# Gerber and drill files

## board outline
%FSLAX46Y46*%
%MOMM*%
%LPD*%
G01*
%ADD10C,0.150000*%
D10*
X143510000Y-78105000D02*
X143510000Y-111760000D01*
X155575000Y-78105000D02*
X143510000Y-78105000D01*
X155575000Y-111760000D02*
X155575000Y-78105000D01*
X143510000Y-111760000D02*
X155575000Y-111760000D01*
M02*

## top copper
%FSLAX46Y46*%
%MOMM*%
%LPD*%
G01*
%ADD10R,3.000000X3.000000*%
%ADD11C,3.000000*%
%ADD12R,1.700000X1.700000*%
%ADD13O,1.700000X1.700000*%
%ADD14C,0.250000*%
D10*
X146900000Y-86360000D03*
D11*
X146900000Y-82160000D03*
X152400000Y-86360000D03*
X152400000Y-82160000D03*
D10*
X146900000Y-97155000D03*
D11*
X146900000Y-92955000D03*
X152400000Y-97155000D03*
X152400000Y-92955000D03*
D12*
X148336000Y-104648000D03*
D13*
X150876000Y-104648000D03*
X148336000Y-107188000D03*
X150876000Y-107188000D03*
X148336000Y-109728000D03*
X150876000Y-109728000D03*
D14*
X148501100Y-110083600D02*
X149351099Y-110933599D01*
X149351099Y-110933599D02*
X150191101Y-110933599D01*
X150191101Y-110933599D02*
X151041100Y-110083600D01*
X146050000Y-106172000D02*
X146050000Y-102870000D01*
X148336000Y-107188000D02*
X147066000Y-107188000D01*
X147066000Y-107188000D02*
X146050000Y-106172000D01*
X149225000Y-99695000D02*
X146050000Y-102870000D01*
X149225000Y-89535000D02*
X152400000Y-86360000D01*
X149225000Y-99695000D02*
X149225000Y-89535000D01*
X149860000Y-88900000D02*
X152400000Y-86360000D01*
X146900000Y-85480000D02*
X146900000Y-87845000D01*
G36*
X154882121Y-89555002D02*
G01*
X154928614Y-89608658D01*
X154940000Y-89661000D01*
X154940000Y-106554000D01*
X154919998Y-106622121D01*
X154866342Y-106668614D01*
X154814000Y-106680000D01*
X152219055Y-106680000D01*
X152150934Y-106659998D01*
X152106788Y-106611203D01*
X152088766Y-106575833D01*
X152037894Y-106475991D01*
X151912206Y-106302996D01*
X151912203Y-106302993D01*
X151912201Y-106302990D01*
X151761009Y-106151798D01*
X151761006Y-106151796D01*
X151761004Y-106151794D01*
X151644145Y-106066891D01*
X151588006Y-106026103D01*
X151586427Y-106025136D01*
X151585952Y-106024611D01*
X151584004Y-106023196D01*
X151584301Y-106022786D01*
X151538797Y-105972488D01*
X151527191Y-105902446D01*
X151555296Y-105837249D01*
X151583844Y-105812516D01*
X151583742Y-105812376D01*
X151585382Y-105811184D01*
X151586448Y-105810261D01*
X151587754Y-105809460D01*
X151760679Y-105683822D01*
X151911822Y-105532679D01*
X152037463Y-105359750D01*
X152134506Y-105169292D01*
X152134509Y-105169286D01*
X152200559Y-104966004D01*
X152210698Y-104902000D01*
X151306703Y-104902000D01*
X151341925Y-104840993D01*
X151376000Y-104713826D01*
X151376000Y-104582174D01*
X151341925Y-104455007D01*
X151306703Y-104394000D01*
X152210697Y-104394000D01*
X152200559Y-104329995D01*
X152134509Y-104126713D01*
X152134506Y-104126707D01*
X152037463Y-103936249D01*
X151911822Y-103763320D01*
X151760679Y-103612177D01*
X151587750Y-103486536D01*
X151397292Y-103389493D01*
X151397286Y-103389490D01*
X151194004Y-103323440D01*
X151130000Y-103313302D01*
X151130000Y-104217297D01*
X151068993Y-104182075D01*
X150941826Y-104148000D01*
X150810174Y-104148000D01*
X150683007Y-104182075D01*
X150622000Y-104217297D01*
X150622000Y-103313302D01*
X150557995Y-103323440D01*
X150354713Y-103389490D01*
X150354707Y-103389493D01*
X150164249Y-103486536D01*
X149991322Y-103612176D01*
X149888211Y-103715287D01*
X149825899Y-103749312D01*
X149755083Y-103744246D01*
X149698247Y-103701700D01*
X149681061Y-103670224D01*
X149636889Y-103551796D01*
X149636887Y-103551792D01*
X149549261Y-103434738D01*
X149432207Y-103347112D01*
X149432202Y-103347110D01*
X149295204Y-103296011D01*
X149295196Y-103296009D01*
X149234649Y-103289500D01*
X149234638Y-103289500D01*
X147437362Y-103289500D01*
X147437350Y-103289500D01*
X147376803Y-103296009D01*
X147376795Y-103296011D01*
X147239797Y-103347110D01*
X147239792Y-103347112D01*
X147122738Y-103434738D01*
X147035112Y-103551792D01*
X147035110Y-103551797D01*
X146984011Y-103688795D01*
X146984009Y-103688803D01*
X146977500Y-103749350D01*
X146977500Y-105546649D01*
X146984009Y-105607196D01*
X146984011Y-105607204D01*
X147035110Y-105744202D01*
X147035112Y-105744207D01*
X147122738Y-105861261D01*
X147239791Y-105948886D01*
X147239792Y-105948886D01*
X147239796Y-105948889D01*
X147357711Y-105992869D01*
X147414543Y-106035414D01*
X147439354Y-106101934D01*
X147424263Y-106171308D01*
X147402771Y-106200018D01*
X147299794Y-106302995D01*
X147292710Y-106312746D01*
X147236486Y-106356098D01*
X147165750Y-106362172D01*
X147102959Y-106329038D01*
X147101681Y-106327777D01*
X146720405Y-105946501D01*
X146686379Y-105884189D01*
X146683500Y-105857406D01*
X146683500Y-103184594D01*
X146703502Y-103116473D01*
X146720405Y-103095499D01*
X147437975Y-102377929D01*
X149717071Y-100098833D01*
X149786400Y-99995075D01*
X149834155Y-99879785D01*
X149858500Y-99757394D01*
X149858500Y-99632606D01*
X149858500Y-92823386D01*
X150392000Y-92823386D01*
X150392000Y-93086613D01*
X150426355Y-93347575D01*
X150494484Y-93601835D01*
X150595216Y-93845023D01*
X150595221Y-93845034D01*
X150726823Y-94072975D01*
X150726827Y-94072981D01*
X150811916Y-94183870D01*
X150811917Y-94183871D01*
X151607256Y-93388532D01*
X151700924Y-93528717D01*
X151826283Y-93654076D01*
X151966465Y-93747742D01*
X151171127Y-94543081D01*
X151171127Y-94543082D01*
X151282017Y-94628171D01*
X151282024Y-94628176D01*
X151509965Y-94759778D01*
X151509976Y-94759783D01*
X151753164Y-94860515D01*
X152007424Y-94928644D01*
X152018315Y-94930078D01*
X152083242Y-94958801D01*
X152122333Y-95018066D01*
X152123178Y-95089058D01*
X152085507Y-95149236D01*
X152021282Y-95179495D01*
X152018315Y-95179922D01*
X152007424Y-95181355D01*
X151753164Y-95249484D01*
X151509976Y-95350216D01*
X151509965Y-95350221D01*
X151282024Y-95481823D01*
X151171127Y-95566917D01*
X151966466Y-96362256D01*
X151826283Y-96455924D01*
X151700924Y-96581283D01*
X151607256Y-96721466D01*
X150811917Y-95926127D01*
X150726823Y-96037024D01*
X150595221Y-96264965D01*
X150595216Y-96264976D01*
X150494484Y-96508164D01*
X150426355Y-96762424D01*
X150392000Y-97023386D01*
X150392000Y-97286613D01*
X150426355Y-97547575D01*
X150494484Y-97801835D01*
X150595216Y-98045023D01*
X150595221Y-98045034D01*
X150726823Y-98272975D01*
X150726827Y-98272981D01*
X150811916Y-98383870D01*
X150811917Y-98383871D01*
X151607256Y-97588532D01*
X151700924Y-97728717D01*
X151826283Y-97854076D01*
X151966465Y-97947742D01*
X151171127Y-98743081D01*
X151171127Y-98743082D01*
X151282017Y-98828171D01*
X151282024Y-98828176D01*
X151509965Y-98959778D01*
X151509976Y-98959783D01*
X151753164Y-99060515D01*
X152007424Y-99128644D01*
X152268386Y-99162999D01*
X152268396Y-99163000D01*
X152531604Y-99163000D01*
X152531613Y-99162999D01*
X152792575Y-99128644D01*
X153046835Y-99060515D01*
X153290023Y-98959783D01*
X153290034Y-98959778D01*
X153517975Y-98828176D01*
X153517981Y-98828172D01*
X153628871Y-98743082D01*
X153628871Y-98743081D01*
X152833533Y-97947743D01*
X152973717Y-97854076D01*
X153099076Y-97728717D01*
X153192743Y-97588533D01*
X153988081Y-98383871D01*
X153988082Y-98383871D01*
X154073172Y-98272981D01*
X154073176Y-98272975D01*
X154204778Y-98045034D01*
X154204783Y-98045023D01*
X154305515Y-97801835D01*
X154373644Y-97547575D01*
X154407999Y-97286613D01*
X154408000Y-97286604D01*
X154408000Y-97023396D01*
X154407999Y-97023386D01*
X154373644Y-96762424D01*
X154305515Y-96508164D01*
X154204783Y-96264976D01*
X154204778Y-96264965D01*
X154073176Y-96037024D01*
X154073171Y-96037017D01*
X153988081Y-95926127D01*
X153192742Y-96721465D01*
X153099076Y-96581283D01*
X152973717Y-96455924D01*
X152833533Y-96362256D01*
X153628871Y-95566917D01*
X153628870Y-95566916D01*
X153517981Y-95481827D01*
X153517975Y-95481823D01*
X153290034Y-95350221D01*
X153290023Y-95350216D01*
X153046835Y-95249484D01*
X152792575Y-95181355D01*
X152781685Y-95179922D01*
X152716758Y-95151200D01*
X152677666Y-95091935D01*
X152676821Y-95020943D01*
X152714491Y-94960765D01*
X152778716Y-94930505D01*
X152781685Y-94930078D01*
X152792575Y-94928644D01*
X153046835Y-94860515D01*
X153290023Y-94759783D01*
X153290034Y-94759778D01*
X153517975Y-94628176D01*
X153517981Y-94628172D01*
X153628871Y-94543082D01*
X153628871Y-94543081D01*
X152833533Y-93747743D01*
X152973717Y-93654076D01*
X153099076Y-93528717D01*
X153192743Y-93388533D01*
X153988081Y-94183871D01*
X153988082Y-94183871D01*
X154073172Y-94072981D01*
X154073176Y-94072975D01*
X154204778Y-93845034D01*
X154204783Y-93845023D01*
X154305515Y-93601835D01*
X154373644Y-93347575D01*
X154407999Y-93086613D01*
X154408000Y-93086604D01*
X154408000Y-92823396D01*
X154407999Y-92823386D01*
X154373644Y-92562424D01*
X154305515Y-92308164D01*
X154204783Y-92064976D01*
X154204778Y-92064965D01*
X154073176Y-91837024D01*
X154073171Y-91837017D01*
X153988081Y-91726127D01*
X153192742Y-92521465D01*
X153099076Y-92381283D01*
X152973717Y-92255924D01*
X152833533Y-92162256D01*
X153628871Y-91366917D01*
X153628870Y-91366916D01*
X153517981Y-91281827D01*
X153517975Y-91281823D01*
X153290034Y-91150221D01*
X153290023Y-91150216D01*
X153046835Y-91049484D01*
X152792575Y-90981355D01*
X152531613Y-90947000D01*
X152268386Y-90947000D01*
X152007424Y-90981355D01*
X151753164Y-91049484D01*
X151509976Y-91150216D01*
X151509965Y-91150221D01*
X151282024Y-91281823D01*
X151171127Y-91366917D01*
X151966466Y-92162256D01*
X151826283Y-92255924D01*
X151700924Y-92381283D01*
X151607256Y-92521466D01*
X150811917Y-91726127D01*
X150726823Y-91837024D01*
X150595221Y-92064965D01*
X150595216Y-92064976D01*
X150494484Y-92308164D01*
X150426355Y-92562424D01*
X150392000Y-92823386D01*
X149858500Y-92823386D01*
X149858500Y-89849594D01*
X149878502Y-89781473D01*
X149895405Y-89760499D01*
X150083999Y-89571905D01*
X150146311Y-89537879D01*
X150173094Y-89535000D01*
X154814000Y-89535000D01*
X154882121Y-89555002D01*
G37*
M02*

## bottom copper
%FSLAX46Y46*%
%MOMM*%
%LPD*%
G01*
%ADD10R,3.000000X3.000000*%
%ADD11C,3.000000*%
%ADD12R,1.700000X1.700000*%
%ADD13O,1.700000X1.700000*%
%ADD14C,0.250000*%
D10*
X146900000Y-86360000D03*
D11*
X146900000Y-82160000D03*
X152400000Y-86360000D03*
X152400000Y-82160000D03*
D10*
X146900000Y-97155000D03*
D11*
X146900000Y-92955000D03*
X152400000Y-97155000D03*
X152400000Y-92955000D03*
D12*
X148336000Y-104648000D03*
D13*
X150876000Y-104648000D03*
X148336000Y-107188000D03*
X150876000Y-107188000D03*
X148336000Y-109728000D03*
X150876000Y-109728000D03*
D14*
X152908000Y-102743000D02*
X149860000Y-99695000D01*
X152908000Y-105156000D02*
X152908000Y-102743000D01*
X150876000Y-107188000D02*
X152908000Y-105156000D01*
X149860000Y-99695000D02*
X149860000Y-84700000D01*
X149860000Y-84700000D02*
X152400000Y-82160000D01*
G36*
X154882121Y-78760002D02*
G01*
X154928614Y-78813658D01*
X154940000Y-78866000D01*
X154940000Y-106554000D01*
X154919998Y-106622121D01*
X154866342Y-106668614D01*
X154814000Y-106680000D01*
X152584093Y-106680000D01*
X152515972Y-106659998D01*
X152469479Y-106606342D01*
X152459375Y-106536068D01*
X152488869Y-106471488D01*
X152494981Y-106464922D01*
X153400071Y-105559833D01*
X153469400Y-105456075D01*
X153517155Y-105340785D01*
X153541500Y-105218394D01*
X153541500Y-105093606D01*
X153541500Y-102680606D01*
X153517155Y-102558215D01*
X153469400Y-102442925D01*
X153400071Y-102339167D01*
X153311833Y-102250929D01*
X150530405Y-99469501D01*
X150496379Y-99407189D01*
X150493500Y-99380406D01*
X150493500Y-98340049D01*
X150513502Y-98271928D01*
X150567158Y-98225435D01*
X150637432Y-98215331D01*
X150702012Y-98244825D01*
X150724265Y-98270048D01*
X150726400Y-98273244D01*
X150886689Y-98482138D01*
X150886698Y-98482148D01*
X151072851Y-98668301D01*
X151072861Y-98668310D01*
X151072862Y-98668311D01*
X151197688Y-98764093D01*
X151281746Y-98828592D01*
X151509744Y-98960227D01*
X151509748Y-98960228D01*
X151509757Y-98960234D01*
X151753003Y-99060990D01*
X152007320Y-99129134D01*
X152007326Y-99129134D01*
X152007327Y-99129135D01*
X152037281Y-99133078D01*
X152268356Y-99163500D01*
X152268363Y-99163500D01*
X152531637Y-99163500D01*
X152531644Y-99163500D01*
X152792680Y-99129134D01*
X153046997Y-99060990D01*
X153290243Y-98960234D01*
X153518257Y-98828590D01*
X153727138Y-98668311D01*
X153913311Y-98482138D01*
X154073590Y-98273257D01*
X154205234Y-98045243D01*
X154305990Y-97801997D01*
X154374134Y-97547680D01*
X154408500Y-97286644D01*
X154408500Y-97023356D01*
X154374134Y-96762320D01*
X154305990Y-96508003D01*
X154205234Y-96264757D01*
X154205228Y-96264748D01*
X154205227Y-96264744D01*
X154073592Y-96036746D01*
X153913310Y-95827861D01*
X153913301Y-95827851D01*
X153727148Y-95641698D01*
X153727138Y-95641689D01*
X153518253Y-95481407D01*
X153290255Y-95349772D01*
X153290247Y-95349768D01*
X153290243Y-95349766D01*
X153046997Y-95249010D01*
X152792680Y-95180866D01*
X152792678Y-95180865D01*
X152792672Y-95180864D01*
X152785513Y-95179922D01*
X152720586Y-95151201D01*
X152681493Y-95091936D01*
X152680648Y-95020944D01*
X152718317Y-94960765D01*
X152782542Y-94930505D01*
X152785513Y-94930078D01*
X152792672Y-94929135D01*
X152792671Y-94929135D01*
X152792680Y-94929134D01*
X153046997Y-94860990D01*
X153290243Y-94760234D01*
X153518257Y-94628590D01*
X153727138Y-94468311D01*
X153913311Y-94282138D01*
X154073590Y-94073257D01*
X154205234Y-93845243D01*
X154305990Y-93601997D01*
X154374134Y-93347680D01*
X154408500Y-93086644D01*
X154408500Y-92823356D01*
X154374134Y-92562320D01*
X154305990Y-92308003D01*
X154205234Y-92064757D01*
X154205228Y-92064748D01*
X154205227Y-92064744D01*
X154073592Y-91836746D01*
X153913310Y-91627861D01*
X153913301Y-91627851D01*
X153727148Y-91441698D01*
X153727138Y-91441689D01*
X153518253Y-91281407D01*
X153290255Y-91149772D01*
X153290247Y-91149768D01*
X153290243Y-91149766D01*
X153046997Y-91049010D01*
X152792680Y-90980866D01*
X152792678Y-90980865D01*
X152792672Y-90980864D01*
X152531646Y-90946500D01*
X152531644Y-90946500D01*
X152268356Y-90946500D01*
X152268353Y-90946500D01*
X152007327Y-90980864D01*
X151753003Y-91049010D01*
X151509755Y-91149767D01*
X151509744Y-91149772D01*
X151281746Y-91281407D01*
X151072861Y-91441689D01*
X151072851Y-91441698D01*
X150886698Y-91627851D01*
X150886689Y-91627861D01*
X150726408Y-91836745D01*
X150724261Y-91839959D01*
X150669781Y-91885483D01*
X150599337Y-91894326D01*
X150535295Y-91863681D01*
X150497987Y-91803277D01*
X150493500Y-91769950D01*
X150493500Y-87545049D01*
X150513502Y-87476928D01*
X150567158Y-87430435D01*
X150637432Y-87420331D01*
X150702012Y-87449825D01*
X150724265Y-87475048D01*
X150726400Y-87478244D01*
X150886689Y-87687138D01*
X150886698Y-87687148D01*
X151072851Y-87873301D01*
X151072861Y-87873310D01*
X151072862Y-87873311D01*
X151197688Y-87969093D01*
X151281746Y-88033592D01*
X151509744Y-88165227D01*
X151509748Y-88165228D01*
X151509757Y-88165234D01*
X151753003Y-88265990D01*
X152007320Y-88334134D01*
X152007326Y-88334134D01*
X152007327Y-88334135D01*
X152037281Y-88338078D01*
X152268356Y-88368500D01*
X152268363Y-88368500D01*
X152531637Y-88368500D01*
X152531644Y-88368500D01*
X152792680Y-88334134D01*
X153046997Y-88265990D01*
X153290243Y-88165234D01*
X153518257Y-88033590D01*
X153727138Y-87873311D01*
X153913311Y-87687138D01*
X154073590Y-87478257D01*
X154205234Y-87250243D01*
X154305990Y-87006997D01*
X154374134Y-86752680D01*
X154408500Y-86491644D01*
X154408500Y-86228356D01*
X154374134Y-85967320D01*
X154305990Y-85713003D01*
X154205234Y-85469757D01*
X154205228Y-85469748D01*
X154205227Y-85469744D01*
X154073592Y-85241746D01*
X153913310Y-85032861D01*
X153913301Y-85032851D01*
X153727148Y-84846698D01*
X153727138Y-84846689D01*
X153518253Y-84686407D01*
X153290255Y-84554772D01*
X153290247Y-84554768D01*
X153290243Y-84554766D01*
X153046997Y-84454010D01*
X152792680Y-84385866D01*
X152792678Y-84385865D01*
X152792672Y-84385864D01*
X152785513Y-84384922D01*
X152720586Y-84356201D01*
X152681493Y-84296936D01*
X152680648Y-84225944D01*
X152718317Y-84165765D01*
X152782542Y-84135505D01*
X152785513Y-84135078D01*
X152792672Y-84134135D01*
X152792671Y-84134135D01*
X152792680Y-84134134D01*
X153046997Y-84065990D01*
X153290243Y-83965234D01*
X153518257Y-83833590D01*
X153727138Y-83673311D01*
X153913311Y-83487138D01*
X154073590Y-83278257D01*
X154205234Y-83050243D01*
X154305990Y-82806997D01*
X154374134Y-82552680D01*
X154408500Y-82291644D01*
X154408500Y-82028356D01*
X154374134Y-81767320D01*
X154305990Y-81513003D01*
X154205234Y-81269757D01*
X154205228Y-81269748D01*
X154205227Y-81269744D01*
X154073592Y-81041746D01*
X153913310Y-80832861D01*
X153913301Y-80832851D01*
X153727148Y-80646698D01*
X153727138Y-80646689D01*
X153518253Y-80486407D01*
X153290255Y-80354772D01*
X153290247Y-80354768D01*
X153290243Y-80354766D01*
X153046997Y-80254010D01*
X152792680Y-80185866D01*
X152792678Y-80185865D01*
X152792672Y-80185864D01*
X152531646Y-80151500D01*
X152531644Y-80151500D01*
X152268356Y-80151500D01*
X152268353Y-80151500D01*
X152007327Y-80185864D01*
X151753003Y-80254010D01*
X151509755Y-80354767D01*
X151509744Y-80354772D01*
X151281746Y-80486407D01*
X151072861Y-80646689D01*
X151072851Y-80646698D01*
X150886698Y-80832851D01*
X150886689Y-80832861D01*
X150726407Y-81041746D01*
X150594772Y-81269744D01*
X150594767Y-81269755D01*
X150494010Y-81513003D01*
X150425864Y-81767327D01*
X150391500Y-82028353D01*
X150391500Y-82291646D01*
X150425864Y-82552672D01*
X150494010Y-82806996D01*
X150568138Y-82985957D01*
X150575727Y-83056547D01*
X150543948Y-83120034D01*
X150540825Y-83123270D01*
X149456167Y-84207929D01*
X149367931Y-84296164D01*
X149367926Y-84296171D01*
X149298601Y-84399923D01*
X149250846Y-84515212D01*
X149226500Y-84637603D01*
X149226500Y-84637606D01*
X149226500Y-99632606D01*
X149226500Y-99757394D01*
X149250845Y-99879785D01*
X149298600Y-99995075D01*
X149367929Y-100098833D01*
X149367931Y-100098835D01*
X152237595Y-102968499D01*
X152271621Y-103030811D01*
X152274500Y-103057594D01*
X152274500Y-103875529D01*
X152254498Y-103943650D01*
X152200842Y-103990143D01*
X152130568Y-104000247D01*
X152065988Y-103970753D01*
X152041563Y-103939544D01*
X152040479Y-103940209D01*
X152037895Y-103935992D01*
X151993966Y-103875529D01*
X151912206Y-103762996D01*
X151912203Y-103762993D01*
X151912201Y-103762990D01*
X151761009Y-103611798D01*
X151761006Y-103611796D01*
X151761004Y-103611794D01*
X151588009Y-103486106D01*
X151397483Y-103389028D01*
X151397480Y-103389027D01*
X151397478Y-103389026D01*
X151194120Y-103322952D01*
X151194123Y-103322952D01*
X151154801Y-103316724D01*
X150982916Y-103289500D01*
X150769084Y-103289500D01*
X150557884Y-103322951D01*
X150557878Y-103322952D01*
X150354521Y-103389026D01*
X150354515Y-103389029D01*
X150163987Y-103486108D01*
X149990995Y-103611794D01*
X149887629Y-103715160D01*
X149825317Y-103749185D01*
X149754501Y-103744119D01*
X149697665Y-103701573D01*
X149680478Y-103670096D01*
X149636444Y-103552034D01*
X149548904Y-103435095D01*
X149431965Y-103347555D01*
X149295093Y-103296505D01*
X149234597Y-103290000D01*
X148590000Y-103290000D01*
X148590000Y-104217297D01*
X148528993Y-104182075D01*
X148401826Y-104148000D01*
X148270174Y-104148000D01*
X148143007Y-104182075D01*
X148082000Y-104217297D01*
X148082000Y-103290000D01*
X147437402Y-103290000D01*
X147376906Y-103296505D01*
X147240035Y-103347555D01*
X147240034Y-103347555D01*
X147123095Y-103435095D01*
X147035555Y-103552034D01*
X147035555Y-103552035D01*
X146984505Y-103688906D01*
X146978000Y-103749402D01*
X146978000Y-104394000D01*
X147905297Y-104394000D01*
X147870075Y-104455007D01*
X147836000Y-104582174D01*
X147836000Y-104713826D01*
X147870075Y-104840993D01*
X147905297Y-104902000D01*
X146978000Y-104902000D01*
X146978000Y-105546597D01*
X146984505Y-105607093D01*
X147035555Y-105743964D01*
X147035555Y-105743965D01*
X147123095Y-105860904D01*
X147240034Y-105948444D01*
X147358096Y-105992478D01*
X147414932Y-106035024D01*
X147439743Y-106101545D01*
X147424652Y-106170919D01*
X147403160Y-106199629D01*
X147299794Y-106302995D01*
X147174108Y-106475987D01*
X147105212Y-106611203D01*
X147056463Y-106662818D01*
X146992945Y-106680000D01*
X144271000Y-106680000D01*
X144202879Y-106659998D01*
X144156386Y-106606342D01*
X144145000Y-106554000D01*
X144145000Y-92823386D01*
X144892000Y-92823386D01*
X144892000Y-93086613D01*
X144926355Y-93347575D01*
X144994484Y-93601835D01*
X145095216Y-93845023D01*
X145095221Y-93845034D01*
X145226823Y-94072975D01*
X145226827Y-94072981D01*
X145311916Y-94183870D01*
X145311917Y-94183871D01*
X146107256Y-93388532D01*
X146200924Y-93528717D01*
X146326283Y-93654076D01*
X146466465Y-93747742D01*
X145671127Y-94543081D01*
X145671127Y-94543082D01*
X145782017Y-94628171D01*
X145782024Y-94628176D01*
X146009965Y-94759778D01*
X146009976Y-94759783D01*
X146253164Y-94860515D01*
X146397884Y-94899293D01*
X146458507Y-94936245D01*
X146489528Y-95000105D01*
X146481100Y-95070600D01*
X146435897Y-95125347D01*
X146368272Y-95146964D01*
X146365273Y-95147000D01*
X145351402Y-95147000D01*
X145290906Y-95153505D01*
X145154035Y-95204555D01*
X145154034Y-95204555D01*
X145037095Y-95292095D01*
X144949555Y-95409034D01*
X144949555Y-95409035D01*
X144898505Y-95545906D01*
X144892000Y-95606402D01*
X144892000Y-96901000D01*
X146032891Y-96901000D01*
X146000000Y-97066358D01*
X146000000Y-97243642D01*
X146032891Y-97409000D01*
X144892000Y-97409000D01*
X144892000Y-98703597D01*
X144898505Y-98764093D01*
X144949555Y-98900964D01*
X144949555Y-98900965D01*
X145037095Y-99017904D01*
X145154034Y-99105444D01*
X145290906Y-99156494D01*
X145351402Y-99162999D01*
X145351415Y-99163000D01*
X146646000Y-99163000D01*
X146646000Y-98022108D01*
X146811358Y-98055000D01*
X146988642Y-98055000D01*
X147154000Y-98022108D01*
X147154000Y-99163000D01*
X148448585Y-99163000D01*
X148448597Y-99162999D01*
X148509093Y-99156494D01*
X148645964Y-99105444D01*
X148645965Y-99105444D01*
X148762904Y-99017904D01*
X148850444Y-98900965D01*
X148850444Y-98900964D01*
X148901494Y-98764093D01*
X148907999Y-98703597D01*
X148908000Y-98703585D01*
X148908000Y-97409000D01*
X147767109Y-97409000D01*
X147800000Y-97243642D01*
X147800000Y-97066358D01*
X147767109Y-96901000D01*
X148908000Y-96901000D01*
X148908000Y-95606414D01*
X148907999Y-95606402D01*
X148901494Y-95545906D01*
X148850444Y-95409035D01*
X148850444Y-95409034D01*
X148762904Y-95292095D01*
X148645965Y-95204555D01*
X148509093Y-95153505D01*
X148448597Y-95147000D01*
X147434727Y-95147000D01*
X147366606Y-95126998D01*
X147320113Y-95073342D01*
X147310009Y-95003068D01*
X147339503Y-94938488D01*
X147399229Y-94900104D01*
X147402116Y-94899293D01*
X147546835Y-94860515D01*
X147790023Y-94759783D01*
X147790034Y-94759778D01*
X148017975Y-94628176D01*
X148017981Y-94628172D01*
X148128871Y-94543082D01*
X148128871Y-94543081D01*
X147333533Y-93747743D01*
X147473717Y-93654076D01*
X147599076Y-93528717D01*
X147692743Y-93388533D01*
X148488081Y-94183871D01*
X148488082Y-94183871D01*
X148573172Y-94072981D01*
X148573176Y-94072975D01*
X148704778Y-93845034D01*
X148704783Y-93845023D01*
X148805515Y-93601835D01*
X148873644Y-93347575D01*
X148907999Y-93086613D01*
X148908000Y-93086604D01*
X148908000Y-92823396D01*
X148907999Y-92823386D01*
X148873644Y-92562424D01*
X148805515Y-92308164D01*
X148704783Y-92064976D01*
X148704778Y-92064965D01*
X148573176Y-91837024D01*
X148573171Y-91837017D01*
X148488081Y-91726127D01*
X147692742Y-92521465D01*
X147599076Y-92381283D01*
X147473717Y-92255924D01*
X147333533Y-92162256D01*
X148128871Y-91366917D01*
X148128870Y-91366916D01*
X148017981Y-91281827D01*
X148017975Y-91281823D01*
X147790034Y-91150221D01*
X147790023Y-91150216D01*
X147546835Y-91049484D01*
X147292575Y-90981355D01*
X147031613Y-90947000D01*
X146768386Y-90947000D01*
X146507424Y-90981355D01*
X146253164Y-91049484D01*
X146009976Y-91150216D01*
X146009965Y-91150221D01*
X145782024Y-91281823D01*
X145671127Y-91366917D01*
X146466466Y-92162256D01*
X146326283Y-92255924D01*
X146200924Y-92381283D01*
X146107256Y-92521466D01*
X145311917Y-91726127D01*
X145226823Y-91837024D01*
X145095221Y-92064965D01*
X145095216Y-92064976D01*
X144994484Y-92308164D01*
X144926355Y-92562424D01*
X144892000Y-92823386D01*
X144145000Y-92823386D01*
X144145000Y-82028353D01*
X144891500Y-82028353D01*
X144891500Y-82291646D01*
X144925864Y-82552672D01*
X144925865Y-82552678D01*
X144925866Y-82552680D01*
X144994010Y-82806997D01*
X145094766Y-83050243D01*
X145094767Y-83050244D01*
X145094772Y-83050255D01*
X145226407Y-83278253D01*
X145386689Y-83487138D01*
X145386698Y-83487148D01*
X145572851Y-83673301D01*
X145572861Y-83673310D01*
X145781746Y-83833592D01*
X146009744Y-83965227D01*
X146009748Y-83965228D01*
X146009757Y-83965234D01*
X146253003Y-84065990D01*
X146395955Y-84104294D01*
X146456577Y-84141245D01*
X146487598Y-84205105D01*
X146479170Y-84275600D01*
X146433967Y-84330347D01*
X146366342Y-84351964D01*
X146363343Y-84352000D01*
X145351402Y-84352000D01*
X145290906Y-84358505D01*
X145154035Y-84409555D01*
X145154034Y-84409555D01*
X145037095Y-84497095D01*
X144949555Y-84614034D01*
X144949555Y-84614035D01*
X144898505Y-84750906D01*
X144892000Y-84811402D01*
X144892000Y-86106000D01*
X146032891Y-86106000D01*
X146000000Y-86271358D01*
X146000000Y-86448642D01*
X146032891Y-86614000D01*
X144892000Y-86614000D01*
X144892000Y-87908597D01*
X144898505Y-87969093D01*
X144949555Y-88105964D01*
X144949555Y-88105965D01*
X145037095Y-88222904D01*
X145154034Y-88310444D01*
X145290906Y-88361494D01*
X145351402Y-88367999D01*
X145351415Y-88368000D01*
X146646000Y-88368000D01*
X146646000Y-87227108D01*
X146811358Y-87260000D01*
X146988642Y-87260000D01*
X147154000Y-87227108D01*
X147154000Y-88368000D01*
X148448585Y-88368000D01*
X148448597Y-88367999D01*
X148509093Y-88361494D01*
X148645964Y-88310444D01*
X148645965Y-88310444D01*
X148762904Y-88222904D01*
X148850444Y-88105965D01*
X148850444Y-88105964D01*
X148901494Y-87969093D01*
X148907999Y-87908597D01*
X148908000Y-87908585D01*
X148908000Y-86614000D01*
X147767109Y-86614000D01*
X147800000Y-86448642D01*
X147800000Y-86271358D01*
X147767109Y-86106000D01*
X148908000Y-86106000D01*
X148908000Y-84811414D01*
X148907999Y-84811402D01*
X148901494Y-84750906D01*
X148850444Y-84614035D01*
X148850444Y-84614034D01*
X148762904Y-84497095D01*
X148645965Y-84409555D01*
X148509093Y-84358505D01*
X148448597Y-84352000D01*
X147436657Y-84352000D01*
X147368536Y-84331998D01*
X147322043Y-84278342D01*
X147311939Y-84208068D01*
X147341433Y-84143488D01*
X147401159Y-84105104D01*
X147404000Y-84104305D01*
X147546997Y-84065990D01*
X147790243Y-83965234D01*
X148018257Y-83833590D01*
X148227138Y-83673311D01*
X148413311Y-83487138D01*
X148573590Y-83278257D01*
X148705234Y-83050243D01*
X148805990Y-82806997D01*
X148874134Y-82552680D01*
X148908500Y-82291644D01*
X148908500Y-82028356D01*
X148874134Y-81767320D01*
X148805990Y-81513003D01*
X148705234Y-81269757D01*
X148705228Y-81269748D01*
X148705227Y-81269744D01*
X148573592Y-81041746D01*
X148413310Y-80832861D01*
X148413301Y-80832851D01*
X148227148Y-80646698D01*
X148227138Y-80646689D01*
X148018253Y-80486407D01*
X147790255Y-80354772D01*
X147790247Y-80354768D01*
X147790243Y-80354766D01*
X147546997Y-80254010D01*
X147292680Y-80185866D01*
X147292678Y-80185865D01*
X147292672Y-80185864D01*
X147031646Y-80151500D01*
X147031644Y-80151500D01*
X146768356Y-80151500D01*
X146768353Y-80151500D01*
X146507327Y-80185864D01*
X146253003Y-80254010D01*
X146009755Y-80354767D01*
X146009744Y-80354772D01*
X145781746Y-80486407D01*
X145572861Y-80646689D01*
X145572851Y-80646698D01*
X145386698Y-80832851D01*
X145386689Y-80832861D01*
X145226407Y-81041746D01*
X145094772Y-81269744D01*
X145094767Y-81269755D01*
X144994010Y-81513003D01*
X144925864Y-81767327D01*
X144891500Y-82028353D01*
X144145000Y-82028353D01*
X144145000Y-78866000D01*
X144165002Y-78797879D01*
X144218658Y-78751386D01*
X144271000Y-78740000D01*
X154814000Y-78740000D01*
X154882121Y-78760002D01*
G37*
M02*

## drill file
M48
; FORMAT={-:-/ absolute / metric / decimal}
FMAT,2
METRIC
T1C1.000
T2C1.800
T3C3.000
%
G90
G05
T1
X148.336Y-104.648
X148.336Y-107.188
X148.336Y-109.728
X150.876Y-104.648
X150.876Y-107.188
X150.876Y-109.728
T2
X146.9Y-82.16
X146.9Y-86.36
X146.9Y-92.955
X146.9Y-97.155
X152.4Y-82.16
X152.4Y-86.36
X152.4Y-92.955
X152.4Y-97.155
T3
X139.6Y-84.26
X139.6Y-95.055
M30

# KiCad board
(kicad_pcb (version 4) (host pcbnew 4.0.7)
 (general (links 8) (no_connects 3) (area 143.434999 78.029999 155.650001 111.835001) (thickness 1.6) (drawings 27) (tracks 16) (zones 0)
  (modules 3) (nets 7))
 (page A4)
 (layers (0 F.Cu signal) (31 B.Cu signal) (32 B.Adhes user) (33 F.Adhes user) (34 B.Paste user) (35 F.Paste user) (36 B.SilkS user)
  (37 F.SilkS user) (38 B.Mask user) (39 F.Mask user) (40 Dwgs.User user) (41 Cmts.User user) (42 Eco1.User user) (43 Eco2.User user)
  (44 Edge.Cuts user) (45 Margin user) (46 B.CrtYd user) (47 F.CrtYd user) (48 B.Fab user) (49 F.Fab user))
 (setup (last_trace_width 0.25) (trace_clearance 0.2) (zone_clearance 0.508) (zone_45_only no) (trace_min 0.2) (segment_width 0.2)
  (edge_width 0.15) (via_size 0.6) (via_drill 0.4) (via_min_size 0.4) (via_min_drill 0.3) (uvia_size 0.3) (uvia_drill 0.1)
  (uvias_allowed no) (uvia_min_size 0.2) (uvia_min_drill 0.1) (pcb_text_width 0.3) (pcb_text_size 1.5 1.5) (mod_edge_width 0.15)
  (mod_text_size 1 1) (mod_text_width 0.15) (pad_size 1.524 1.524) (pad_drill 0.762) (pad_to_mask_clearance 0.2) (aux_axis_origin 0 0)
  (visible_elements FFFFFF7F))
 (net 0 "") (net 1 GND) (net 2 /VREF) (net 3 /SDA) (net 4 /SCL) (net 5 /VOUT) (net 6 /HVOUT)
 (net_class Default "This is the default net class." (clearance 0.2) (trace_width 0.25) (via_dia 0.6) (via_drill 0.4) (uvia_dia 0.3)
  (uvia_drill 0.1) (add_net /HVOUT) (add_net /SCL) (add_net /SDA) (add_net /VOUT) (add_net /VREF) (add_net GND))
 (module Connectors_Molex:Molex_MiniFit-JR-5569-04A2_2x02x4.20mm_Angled (layer F.Cu) (at 146.9 86.36 90)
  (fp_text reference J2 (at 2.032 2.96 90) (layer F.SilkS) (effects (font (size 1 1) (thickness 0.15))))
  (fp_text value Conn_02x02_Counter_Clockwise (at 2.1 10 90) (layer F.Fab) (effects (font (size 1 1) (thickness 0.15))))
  (pad 1 thru_hole rect (at 0 0 90) (size 3 3) (drill 1.8) (layers *.Cu *.Mask) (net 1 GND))
  (pad 2 thru_hole circle (at 4.2 0 90) (size 3 3) (drill 1.8) (layers *.Cu *.Mask) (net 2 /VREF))
  (pad 3 thru_hole circle (at 0 5.5 90) (size 3 3) (drill 1.8) (layers *.Cu *.Mask) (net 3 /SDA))
  (pad 4 thru_hole circle (at 4.2 5.5 90) (size 3 3) (drill 1.8) (layers *.Cu *.Mask) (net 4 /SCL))
  (pad "" np_thru_hole circle (at 2.1 -7.3 90) (size 3 3) (drill 3) (layers *.Cu *.Mask)))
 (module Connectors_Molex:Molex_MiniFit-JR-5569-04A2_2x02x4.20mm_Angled (layer F.Cu) (at 146.9 97.155 90)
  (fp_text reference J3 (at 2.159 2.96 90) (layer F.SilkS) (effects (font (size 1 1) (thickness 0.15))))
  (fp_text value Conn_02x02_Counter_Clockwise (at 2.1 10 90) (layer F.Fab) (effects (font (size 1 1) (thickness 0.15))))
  (pad 1 thru_hole rect (at 0 0 90) (size 3 3) (drill 1.8) (layers *.Cu *.Mask) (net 1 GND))
  (pad 2 thru_hole circle (at 4.2 0 90) (size 3 3) (drill 1.8) (layers *.Cu *.Mask) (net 1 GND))
  (pad 3 thru_hole circle (at 0 5.5 90) (size 3 3) (drill 1.8) (layers *.Cu *.Mask) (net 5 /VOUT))
  (pad 4 thru_hole circle (at 4.2 5.5 90) (size 3 3) (drill 1.8) (layers *.Cu *.Mask) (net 5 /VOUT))
  (pad "" np_thru_hole circle (at 2.1 -7.3 90) (size 3 3) (drill 3) (layers *.Cu *.Mask)))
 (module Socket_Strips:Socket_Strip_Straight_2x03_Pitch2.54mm (layer B.Cu) (at 148.336 104.648 180)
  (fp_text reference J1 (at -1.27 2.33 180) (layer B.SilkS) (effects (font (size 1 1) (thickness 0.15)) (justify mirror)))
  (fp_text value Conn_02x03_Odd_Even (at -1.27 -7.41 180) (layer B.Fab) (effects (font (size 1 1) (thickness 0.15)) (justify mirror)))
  (pad 1 thru_hole rect (at 0 0 180) (size 1.7 1.7) (drill 1) (layers *.Cu *.Mask) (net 1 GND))
  (pad 2 thru_hole oval (at -2.54 0 180) (size 1.7 1.7) (drill 1) (layers *.Cu *.Mask) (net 5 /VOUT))
  (pad 3 thru_hole oval (at 0 -2.54 180) (size 1.7 1.7) (drill 1) (layers *.Cu *.Mask) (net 3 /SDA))
  (pad 4 thru_hole oval (at -2.54 -2.54 180) (size 1.7 1.7) (drill 1) (layers *.Cu *.Mask) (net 4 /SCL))
  (pad 5 thru_hole oval (at 0 -5.08 180) (size 1.7 1.7) (drill 1) (layers *.Cu *.Mask) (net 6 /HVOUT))
  (pad 6 thru_hole oval (at -2.54 -5.08 180) (size 1.7 1.7) (drill 1) (layers *.Cu *.Mask) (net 6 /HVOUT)))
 (gr_line (start 143.51 78.105) (end 143.51 111.76) (layer Edge.Cuts) (width 0.15))
 (gr_line (start 155.575 78.105) (end 143.51 78.105) (layer Edge.Cuts) (width 0.15))
 (gr_line (start 155.575 111.76) (end 155.575 78.105) (layer Edge.Cuts) (width 0.15))
 (gr_line (start 143.51 111.76) (end 155.575 111.76) (layer Edge.Cuts) (width 0.15))
 (segment (start 152.908 102.743) (end 149.86 99.695) (width 0.25) (layer B.Cu) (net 4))
 (segment (start 152.908 105.156) (end 152.908 102.743) (width 0.25) (layer B.Cu) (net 4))
 (segment (start 150.876 107.188) (end 152.908 105.156) (width 0.25) (layer B.Cu) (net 4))
 (segment (start 149.86 99.695) (end 149.86 84.7) (width 0.25) (layer B.Cu) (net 4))
 (segment (start 149.86 84.7) (end 152.4 82.16) (width 0.25) (layer B.Cu) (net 4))
 (segment (start 148.5011 110.0836) (end 149.351099 110.933599) (width 0.25) (layer F.Cu) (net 6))
 (segment (start 149.351099 110.933599) (end 150.191101 110.933599) (width 0.25) (layer F.Cu) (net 6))
 (segment (start 150.191101 110.933599) (end 151.0411 110.0836) (width 0.25) (layer F.Cu) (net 6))
 (segment (start 146.05 106.172) (end 146.05 102.87) (width 0.25) (layer F.Cu) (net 3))
 (segment (start 148.336 107.188) (end 147.066 107.188) (width 0.25) (layer F.Cu) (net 3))
 (segment (start 147.066 107.188) (end 146.05 106.172) (width 0.25) (layer F.Cu) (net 3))
 (segment (start 149.225 99.695) (end 146.05 102.87) (width 0.25) (layer F.Cu) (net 3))
 (segment (start 149.225 89.535) (end 152.4 86.36) (width 0.25) (layer F.Cu) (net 3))
 (segment (start 149.225 99.695) (end 149.225 89.535) (width 0.25) (layer F.Cu) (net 3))
 (segment (start 149.86 88.9) (end 152.4 86.36) (width 0.25) (layer F.Cu) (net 3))
 (segment (start 146.9 85.48) (end 146.9 87.845) (width 0.25) (layer F.Cu) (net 1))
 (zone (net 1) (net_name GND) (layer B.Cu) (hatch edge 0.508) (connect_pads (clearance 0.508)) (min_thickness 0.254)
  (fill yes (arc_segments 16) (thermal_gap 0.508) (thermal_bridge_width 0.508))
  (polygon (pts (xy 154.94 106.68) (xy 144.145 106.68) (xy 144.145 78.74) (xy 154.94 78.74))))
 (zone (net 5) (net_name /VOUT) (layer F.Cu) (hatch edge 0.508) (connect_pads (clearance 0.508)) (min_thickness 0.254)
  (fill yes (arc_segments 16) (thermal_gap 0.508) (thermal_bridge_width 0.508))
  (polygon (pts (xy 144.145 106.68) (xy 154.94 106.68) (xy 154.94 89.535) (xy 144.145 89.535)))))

